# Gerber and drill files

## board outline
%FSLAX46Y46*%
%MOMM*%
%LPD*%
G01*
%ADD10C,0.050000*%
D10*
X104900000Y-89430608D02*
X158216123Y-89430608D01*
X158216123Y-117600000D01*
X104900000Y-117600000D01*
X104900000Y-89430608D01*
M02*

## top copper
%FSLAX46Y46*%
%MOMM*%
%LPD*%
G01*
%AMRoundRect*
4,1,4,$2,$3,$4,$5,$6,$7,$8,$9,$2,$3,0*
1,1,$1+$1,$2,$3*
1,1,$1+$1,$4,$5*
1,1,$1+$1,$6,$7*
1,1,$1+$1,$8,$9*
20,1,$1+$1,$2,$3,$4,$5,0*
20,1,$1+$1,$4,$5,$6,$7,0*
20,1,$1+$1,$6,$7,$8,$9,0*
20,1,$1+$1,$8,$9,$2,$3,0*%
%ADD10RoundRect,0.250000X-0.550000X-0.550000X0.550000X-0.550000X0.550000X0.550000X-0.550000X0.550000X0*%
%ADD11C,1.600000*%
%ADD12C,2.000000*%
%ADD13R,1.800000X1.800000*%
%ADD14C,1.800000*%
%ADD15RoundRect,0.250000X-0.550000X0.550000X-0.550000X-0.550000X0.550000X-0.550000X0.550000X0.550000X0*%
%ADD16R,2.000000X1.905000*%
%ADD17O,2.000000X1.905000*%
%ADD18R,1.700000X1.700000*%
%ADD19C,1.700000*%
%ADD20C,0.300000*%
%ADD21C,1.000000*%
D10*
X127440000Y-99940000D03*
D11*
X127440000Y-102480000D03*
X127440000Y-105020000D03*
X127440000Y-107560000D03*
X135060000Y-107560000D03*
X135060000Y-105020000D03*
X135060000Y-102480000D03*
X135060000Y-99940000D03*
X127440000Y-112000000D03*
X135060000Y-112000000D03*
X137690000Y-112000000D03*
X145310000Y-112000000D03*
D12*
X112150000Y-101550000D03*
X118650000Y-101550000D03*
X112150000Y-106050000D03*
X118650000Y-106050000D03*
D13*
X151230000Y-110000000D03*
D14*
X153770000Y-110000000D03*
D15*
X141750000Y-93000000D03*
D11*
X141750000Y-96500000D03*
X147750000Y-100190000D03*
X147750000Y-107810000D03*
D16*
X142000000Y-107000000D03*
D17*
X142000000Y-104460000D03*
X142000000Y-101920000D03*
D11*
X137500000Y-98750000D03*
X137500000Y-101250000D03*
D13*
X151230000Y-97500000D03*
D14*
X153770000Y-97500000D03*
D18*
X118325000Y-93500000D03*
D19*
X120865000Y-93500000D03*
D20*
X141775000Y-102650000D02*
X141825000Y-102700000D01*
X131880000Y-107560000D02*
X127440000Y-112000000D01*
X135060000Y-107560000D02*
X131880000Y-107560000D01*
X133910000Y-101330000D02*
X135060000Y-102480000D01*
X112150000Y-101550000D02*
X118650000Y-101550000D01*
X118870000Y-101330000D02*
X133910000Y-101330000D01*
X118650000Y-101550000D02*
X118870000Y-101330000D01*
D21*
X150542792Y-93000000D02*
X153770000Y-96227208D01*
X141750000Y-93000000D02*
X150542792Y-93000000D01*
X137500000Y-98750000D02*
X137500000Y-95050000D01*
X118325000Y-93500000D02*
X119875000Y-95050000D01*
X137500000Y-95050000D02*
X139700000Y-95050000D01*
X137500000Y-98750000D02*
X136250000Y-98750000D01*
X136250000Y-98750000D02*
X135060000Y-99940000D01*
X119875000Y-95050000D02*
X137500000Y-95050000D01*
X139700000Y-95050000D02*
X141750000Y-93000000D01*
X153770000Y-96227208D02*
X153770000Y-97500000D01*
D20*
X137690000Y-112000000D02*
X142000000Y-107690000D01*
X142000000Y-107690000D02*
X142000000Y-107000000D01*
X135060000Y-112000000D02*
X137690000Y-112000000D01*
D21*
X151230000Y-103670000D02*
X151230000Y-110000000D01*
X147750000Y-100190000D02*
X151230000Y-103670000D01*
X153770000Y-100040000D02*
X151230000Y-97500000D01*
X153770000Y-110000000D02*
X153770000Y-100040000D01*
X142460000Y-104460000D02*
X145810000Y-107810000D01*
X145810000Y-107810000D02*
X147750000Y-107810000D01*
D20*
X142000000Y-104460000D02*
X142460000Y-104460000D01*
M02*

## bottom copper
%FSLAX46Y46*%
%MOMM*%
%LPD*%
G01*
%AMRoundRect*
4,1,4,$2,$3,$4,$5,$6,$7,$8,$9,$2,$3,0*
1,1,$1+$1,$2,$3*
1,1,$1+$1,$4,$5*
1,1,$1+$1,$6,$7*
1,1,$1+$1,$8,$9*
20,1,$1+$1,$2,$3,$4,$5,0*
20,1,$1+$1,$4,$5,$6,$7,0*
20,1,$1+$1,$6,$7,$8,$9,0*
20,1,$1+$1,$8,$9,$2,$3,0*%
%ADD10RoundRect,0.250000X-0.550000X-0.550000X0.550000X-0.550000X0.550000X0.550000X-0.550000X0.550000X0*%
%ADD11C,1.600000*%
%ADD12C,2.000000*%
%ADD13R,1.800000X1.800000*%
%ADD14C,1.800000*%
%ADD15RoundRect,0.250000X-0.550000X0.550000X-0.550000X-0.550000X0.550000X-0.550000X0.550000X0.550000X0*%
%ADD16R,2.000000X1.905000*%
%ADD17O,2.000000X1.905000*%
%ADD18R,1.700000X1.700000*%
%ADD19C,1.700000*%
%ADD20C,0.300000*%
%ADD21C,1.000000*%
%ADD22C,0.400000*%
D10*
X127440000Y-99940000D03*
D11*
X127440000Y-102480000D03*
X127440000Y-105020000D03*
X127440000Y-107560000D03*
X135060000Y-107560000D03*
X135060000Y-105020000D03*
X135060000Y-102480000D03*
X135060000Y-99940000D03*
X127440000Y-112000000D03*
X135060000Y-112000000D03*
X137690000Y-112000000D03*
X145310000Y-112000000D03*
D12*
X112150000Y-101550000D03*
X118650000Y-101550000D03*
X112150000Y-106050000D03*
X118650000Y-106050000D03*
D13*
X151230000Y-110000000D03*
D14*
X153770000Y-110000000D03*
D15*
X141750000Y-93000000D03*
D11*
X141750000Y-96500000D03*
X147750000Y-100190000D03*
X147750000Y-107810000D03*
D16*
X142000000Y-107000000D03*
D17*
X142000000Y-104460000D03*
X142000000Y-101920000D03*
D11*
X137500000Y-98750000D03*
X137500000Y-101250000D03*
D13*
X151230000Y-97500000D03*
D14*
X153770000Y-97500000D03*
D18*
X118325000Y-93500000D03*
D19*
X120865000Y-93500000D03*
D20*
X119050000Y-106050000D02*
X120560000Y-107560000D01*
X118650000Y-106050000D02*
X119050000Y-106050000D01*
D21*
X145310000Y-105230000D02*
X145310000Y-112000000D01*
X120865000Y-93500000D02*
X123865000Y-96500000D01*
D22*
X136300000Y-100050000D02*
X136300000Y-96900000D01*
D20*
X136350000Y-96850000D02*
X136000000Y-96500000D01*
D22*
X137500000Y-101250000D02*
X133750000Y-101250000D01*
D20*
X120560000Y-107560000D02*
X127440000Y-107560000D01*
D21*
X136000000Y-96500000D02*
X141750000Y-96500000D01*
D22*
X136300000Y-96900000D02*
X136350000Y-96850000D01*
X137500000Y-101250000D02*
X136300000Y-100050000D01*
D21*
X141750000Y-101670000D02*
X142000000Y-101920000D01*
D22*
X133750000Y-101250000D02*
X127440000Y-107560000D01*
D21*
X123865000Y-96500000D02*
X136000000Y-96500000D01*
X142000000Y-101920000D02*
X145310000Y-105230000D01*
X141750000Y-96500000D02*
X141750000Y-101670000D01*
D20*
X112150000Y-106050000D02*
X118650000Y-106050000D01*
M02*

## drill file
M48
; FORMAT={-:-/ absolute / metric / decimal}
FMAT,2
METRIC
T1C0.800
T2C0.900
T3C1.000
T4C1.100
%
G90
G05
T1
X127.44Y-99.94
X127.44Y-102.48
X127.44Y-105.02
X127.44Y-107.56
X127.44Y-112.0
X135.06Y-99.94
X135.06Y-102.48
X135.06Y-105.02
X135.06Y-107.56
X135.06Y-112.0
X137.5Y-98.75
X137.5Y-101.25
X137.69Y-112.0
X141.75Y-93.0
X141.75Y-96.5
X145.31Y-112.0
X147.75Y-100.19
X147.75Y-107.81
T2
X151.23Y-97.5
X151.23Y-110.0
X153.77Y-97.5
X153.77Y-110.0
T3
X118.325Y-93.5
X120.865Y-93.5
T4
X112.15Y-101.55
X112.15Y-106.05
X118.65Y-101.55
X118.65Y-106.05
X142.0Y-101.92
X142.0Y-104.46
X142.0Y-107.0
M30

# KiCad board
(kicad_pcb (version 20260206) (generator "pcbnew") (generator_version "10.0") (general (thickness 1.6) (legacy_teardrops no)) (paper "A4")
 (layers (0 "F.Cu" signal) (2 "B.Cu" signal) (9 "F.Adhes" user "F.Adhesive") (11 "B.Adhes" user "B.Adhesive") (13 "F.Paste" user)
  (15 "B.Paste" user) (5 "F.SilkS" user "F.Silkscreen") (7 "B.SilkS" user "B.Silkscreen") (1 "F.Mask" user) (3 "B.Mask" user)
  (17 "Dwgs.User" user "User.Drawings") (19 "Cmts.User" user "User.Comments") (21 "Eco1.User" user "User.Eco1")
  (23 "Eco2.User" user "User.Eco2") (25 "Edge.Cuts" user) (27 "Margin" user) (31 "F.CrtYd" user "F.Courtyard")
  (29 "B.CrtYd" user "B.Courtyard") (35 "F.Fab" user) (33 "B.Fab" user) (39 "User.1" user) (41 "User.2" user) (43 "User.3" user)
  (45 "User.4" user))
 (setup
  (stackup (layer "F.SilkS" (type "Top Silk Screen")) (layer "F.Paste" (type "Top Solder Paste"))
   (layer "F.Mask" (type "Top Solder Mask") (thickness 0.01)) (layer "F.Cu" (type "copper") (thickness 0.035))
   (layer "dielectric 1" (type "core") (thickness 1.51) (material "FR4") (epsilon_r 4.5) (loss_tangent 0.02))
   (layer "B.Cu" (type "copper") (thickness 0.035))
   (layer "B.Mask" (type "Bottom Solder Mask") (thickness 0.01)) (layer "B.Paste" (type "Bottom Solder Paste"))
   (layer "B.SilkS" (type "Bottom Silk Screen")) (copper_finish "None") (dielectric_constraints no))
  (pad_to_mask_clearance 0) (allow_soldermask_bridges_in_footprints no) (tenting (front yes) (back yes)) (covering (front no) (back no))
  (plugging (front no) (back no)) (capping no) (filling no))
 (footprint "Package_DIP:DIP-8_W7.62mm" (layer "F.Cu") (at 127.44 99.94)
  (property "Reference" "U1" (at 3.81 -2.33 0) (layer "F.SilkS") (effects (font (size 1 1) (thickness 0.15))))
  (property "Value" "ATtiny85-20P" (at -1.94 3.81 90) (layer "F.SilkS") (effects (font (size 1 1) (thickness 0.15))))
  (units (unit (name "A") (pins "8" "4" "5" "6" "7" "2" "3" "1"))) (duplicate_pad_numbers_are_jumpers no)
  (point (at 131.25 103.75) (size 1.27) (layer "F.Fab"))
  (pad "1" thru_hole roundrect (at 0 0) (size 1.6 1.6) (drill 0.8) (layers "*.Cu" "*.Mask") (remove_unused_layers no)
   (roundrect_rratio 0.15625) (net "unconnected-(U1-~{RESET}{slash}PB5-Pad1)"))
  (pad "2" thru_hole circle (at 0 2.54) (size 1.6 1.6) (drill 0.8) (layers "*.Cu" "*.Mask") (remove_unused_layers no)
   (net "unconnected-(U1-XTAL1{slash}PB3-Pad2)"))
  (pad "3" thru_hole circle (at 0 5.08) (size 1.6 1.6) (drill 0.8) (layers "*.Cu" "*.Mask") (remove_unused_layers no)
   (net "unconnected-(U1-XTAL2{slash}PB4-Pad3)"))
  (pad "4" thru_hole circle (at 0 7.62) (size 1.6 1.6) (drill 0.8) (layers "*.Cu" "*.Mask") (remove_unused_layers no) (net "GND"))
  (pad "5" thru_hole circle (at 7.62 7.62) (size 1.6 1.6) (drill 0.8) (layers "*.Cu" "*.Mask") (remove_unused_layers no)
   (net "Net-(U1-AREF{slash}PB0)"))
  (pad "6" thru_hole circle (at 7.62 5.08) (size 1.6 1.6) (drill 0.8) (layers "*.Cu" "*.Mask") (remove_unused_layers no)
   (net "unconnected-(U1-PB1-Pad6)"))
  (pad "7" thru_hole circle (at 7.62 2.54) (size 1.6 1.6) (drill 0.8) (layers "*.Cu" "*.Mask") (remove_unused_layers no)
   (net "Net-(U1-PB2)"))
  (pad "8" thru_hole circle (at 7.62 0) (size 1.6 1.6) (drill 0.8) (layers "*.Cu" "*.Mask") (remove_unused_layers no) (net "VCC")))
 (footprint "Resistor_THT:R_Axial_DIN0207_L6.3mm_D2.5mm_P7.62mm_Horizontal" (layer "F.Cu") (at 127.44 112)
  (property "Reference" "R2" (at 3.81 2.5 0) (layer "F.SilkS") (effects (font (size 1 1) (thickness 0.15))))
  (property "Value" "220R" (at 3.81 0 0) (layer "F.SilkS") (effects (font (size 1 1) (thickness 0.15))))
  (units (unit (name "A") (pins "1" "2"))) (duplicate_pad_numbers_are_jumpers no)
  (pad "1" thru_hole circle (at 0 0) (size 1.6 1.6) (drill 0.8) (layers "*.Cu" "*.Mask") (remove_unused_layers no)
   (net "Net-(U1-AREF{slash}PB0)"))
  (pad "2" thru_hole circle (at 7.62 0) (size 1.6 1.6) (drill 0.8) (layers "*.Cu" "*.Mask") (remove_unused_layers no) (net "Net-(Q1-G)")))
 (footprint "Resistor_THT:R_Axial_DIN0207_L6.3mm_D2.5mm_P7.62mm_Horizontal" (layer "F.Cu") (at 137.69 112)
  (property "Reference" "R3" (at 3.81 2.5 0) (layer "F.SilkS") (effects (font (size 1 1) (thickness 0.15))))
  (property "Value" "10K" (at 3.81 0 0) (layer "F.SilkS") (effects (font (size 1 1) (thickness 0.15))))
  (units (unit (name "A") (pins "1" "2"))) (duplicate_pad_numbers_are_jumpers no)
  (pad "1" thru_hole circle (at 0 0) (size 1.6 1.6) (drill 0.8) (layers "*.Cu" "*.Mask") (remove_unused_layers no) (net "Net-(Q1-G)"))
  (pad "2" thru_hole circle (at 7.62 0) (size 1.6 1.6) (drill 0.8) (layers "*.Cu" "*.Mask") (remove_unused_layers no) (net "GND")))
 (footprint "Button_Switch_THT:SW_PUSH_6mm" (layer "F.Cu") (at 112.15 101.55)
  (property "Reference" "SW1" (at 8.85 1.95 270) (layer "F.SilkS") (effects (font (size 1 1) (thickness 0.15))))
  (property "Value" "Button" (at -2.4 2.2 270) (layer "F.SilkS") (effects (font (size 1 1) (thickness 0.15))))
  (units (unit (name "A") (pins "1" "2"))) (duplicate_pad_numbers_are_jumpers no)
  (pad "1" thru_hole circle (at 0 0 90) (size 2 2) (drill 1.1) (layers "*.Cu" "*.Mask") (remove_unused_layers no) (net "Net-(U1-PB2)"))
  (pad "1" thru_hole circle (at 6.5 0 90) (size 2 2) (drill 1.1) (layers "*.Cu" "*.Mask") (remove_unused_layers no) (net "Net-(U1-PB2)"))
  (pad "2" thru_hole circle (at 0 4.5 90) (size 2 2) (drill 1.1) (layers "*.Cu" "*.Mask") (remove_unused_layers no) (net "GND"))
  (pad "2" thru_hole circle (at 6.5 4.5 90) (size 2 2) (drill 1.1) (layers "*.Cu" "*.Mask") (remove_unused_layers no) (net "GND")))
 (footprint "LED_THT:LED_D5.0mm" (layer "F.Cu") (at 151.23 110)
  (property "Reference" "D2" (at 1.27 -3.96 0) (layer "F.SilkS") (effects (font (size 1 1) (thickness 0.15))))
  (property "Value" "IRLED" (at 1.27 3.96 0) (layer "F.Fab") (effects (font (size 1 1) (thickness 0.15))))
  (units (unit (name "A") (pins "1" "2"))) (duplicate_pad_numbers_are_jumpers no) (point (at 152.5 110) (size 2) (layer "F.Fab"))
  (pad "1" thru_hole rect (at 0 0) (size 1.8 1.8) (drill 0.9) (layers "*.Cu" "*.Mask") (remove_unused_layers no) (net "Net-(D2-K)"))
  (pad "2" thru_hole circle (at 2.54 0) (size 1.8 1.8) (drill 0.9) (layers "*.Cu" "*.Mask") (remove_unused_layers no) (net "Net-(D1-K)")))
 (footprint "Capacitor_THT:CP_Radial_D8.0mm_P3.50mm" (layer "F.Cu") (at 141.75 93 -90)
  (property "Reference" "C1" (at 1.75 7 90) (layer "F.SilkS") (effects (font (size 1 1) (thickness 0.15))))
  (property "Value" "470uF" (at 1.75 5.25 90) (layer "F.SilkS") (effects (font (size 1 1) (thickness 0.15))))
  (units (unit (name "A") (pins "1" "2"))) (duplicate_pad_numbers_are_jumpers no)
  (pad "1" thru_hole roundrect (at 0 0 270) (size 1.6 1.6) (drill 0.8) (layers "*.Cu" "*.Mask") (remove_unused_layers no)
   (roundrect_rratio 0.15625) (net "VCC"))
  (pad "2" thru_hole circle (at 3.5 0 270) (size 1.6 1.6) (drill 0.8) (layers "*.Cu" "*.Mask") (remove_unused_layers no) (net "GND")))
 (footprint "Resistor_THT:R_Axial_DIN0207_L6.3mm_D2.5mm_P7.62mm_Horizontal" (layer "F.Cu") (at 147.75 100.19 -90)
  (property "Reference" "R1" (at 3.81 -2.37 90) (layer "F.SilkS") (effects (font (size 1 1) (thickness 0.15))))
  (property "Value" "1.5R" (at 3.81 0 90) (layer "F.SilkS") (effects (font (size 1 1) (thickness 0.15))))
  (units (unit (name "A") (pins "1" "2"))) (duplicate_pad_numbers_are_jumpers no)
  (pad "1" thru_hole circle (at 0 0 270) (size 1.6 1.6) (drill 0.8) (layers "*.Cu" "*.Mask") (remove_unused_layers no) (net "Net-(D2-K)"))
  (pad "2" thru_hole circle (at 7.62 0 270) (size 1.6 1.6) (drill 0.8) (layers "*.Cu" "*.Mask") (remove_unused_layers no) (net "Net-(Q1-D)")))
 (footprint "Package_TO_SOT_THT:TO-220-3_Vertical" (layer "F.Cu") (at 142 107 90)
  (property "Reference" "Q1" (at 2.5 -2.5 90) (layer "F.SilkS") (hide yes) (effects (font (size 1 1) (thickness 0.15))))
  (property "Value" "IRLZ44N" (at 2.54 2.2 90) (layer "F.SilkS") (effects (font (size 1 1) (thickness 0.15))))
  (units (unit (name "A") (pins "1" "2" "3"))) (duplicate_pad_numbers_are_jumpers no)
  (pad "1" thru_hole rect (at 0 0 90) (size 1.905 2) (drill 1.1) (layers "*.Cu" "*.Mask") (remove_unused_layers no) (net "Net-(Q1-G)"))
  (pad "2" thru_hole oval (at 2.54 0 90) (size 1.905 2) (drill 1.1) (layers "*.Cu" "*.Mask") (remove_unused_layers no) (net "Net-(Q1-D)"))
  (pad "3" thru_hole oval (at 5.08 0 90) (size 1.905 2) (drill 1.1) (layers "*.Cu" "*.Mask") (remove_unused_layers no) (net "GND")))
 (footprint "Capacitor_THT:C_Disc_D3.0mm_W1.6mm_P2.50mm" (layer "F.Cu") (at 137.5 98.75 -90)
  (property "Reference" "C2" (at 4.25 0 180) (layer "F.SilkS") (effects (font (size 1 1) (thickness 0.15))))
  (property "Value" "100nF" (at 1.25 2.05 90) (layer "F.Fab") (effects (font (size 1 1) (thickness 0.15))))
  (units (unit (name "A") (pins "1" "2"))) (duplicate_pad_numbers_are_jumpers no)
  (pad "1" thru_hole circle (at 0 0 270) (size 1.6 1.6) (drill 0.8) (layers "*.Cu" "*.Mask") (remove_unused_layers no) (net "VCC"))
  (pad "2" thru_hole circle (at 2.5 0 270) (size 1.6 1.6) (drill 0.8) (layers "*.Cu" "*.Mask") (remove_unused_layers no) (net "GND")))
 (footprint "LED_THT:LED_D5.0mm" (layer "F.Cu") (at 151.23 97.5)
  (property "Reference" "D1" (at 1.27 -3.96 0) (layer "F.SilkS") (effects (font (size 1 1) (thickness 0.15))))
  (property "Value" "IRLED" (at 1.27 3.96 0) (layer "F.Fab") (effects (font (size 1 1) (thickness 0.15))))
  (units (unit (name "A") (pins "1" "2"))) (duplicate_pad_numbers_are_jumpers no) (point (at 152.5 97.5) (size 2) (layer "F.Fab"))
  (pad "1" thru_hole rect (at 0 0) (size 1.8 1.8) (drill 0.9) (layers "*.Cu" "*.Mask") (remove_unused_layers no) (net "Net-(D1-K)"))
  (pad "2" thru_hole circle (at 2.54 0) (size 1.8 1.8) (drill 0.9) (layers "*.Cu" "*.Mask") (remove_unused_layers no) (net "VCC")))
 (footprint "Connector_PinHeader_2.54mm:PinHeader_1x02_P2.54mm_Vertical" (layer "F.Cu") (at 118.325 93.5 90)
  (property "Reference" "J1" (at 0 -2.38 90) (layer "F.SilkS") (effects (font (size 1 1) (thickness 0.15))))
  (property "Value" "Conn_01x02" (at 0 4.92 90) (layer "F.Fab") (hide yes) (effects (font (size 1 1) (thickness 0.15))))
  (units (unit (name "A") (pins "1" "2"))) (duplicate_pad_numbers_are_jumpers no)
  (pad "1" thru_hole rect (at 0 0 90) (size 1.7 1.7) (drill 1) (layers "*.Cu" "*.Mask") (remove_unused_layers no) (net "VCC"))
  (pad "2" thru_hole circle (at 0 2.54 90) (size 1.7 1.7) (drill 1) (layers "*.Cu" "*.Mask") (remove_unused_layers no) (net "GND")))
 (gr_rect (start 104.9 89.430608) (end 158.216123 117.6) (stroke (width 0.05) (type default)) (fill no) (layer "Edge.Cuts"))
 (segment (start 141.775 102.65) (end 141.825 102.7) (width 0.3) (layer "F.Cu") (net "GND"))
 (segment (start 119.05 106.05) (end 120.56 107.56) (width 0.3) (layer "B.Cu") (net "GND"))
 (segment (start 118.65 106.05) (end 119.05 106.05) (width 0.3) (layer "B.Cu") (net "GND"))
 (segment (start 145.31 105.23) (end 145.31 112) (width 1) (layer "B.Cu") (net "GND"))
 (segment (start 120.865 93.5) (end 123.865 96.5) (width 1) (layer "B.Cu") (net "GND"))
 (segment (start 136.3 100.05) (end 136.3 96.9) (width 0.4) (layer "B.Cu") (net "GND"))
 (segment (start 136.35 96.85) (end 136 96.5) (width 0.3) (layer "B.Cu") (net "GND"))
 (segment (start 137.5 101.25) (end 133.75 101.25) (width 0.4) (layer "B.Cu") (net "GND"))
 (segment (start 120.56 107.56) (end 127.44 107.56) (width 0.3) (layer "B.Cu") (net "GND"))
 (segment (start 136 96.5) (end 141.75 96.5) (width 1) (layer "B.Cu") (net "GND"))
 (segment (start 136.3 96.9) (end 136.35 96.85) (width 0.4) (layer "B.Cu") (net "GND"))
 (segment (start 137.5 101.25) (end 136.3 100.05) (width 0.4) (layer "B.Cu") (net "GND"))
 (segment (start 141.75 101.67) (end 142 101.92) (width 1) (layer "B.Cu") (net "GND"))
 (segment (start 133.75 101.25) (end 127.44 107.56) (width 0.4) (layer "B.Cu") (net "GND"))
 (segment (start 123.865 96.5) (end 136 96.5) (width 1) (layer "B.Cu") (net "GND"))
 (segment (start 142 101.92) (end 145.31 105.23) (width 1) (layer "B.Cu") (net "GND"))
 (segment (start 141.75 96.5) (end 141.75 101.67) (width 1) (layer "B.Cu") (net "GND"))
 (segment (start 112.15 106.05) (end 118.65 106.05) (width 0.3) (layer "B.Cu") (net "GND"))
 (segment (start 131.88 107.56) (end 127.44 112) (width 0.3) (layer "F.Cu") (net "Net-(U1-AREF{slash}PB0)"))
 (segment (start 135.06 107.56) (end 131.88 107.56) (width 0.3) (layer "F.Cu") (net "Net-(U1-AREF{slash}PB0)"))
 (segment (start 133.91 101.33) (end 135.06 102.48) (width 0.3) (layer "F.Cu") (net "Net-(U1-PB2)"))
 (segment (start 112.15 101.55) (end 118.65 101.55) (width 0.3) (layer "F.Cu") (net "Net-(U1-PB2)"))
 (segment (start 118.87 101.33) (end 133.91 101.33) (width 0.3) (layer "F.Cu") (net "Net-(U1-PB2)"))
 (segment (start 118.65 101.55) (end 118.87 101.33) (width 0.3) (layer "F.Cu") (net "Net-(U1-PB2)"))
 (segment (start 150.542792 93) (end 153.77 96.227208) (width 1) (layer "F.Cu") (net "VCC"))
 (segment (start 141.75 93) (end 150.542792 93) (width 1) (layer "F.Cu") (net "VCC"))
 (segment (start 137.5 98.75) (end 137.5 95.05) (width 1) (layer "F.Cu") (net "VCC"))
 (segment (start 118.325 93.5) (end 119.875 95.05) (width 1) (layer "F.Cu") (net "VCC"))
 (segment (start 137.5 95.05) (end 139.7 95.05) (width 1) (layer "F.Cu") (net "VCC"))
 (segment (start 137.5 98.75) (end 136.25 98.75) (width 1) (layer "F.Cu") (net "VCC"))
 (segment (start 136.25 98.75) (end 135.06 99.94) (width 1) (layer "F.Cu") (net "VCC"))
 (segment (start 119.875 95.05) (end 137.5 95.05) (width 1) (layer "F.Cu") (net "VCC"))
 (segment (start 139.7 95.05) (end 141.75 93) (width 1) (layer "F.Cu") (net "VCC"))
 (segment (start 153.77 96.227208) (end 153.77 97.5) (width 1) (layer "F.Cu") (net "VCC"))
 (segment (start 137.69 112) (end 142 107.69) (width 0.3) (layer "F.Cu") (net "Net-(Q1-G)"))
 (segment (start 142 107.69) (end 142 107) (width 0.3) (layer "F.Cu") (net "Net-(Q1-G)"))
 (segment (start 135.06 112) (end 137.69 112) (width 0.3) (layer "F.Cu") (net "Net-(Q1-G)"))
 (segment (start 151.23 103.67) (end 151.23 110) (width 1) (layer "F.Cu") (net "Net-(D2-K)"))
 (segment (start 147.75 100.19) (end 151.23 103.67) (width 1) (layer "F.Cu") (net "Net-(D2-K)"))
 (segment (start 153.77 100.04) (end 151.23 97.5) (width 1) (layer "F.Cu") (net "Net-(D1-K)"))
 (segment (start 153.77 110) (end 153.77 100.04) (width 1) (layer "F.Cu") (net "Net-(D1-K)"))
 (segment (start 142.46 104.46) (end 145.81 107.81) (width 1) (layer "F.Cu") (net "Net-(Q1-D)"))
 (segment (start 145.81 107.81) (end 147.75 107.81) (width 1) (layer "F.Cu") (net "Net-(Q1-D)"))
 (segment (start 142 104.46) (end 142.46 104.46) (width 0.3) (layer "F.Cu") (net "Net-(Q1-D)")))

